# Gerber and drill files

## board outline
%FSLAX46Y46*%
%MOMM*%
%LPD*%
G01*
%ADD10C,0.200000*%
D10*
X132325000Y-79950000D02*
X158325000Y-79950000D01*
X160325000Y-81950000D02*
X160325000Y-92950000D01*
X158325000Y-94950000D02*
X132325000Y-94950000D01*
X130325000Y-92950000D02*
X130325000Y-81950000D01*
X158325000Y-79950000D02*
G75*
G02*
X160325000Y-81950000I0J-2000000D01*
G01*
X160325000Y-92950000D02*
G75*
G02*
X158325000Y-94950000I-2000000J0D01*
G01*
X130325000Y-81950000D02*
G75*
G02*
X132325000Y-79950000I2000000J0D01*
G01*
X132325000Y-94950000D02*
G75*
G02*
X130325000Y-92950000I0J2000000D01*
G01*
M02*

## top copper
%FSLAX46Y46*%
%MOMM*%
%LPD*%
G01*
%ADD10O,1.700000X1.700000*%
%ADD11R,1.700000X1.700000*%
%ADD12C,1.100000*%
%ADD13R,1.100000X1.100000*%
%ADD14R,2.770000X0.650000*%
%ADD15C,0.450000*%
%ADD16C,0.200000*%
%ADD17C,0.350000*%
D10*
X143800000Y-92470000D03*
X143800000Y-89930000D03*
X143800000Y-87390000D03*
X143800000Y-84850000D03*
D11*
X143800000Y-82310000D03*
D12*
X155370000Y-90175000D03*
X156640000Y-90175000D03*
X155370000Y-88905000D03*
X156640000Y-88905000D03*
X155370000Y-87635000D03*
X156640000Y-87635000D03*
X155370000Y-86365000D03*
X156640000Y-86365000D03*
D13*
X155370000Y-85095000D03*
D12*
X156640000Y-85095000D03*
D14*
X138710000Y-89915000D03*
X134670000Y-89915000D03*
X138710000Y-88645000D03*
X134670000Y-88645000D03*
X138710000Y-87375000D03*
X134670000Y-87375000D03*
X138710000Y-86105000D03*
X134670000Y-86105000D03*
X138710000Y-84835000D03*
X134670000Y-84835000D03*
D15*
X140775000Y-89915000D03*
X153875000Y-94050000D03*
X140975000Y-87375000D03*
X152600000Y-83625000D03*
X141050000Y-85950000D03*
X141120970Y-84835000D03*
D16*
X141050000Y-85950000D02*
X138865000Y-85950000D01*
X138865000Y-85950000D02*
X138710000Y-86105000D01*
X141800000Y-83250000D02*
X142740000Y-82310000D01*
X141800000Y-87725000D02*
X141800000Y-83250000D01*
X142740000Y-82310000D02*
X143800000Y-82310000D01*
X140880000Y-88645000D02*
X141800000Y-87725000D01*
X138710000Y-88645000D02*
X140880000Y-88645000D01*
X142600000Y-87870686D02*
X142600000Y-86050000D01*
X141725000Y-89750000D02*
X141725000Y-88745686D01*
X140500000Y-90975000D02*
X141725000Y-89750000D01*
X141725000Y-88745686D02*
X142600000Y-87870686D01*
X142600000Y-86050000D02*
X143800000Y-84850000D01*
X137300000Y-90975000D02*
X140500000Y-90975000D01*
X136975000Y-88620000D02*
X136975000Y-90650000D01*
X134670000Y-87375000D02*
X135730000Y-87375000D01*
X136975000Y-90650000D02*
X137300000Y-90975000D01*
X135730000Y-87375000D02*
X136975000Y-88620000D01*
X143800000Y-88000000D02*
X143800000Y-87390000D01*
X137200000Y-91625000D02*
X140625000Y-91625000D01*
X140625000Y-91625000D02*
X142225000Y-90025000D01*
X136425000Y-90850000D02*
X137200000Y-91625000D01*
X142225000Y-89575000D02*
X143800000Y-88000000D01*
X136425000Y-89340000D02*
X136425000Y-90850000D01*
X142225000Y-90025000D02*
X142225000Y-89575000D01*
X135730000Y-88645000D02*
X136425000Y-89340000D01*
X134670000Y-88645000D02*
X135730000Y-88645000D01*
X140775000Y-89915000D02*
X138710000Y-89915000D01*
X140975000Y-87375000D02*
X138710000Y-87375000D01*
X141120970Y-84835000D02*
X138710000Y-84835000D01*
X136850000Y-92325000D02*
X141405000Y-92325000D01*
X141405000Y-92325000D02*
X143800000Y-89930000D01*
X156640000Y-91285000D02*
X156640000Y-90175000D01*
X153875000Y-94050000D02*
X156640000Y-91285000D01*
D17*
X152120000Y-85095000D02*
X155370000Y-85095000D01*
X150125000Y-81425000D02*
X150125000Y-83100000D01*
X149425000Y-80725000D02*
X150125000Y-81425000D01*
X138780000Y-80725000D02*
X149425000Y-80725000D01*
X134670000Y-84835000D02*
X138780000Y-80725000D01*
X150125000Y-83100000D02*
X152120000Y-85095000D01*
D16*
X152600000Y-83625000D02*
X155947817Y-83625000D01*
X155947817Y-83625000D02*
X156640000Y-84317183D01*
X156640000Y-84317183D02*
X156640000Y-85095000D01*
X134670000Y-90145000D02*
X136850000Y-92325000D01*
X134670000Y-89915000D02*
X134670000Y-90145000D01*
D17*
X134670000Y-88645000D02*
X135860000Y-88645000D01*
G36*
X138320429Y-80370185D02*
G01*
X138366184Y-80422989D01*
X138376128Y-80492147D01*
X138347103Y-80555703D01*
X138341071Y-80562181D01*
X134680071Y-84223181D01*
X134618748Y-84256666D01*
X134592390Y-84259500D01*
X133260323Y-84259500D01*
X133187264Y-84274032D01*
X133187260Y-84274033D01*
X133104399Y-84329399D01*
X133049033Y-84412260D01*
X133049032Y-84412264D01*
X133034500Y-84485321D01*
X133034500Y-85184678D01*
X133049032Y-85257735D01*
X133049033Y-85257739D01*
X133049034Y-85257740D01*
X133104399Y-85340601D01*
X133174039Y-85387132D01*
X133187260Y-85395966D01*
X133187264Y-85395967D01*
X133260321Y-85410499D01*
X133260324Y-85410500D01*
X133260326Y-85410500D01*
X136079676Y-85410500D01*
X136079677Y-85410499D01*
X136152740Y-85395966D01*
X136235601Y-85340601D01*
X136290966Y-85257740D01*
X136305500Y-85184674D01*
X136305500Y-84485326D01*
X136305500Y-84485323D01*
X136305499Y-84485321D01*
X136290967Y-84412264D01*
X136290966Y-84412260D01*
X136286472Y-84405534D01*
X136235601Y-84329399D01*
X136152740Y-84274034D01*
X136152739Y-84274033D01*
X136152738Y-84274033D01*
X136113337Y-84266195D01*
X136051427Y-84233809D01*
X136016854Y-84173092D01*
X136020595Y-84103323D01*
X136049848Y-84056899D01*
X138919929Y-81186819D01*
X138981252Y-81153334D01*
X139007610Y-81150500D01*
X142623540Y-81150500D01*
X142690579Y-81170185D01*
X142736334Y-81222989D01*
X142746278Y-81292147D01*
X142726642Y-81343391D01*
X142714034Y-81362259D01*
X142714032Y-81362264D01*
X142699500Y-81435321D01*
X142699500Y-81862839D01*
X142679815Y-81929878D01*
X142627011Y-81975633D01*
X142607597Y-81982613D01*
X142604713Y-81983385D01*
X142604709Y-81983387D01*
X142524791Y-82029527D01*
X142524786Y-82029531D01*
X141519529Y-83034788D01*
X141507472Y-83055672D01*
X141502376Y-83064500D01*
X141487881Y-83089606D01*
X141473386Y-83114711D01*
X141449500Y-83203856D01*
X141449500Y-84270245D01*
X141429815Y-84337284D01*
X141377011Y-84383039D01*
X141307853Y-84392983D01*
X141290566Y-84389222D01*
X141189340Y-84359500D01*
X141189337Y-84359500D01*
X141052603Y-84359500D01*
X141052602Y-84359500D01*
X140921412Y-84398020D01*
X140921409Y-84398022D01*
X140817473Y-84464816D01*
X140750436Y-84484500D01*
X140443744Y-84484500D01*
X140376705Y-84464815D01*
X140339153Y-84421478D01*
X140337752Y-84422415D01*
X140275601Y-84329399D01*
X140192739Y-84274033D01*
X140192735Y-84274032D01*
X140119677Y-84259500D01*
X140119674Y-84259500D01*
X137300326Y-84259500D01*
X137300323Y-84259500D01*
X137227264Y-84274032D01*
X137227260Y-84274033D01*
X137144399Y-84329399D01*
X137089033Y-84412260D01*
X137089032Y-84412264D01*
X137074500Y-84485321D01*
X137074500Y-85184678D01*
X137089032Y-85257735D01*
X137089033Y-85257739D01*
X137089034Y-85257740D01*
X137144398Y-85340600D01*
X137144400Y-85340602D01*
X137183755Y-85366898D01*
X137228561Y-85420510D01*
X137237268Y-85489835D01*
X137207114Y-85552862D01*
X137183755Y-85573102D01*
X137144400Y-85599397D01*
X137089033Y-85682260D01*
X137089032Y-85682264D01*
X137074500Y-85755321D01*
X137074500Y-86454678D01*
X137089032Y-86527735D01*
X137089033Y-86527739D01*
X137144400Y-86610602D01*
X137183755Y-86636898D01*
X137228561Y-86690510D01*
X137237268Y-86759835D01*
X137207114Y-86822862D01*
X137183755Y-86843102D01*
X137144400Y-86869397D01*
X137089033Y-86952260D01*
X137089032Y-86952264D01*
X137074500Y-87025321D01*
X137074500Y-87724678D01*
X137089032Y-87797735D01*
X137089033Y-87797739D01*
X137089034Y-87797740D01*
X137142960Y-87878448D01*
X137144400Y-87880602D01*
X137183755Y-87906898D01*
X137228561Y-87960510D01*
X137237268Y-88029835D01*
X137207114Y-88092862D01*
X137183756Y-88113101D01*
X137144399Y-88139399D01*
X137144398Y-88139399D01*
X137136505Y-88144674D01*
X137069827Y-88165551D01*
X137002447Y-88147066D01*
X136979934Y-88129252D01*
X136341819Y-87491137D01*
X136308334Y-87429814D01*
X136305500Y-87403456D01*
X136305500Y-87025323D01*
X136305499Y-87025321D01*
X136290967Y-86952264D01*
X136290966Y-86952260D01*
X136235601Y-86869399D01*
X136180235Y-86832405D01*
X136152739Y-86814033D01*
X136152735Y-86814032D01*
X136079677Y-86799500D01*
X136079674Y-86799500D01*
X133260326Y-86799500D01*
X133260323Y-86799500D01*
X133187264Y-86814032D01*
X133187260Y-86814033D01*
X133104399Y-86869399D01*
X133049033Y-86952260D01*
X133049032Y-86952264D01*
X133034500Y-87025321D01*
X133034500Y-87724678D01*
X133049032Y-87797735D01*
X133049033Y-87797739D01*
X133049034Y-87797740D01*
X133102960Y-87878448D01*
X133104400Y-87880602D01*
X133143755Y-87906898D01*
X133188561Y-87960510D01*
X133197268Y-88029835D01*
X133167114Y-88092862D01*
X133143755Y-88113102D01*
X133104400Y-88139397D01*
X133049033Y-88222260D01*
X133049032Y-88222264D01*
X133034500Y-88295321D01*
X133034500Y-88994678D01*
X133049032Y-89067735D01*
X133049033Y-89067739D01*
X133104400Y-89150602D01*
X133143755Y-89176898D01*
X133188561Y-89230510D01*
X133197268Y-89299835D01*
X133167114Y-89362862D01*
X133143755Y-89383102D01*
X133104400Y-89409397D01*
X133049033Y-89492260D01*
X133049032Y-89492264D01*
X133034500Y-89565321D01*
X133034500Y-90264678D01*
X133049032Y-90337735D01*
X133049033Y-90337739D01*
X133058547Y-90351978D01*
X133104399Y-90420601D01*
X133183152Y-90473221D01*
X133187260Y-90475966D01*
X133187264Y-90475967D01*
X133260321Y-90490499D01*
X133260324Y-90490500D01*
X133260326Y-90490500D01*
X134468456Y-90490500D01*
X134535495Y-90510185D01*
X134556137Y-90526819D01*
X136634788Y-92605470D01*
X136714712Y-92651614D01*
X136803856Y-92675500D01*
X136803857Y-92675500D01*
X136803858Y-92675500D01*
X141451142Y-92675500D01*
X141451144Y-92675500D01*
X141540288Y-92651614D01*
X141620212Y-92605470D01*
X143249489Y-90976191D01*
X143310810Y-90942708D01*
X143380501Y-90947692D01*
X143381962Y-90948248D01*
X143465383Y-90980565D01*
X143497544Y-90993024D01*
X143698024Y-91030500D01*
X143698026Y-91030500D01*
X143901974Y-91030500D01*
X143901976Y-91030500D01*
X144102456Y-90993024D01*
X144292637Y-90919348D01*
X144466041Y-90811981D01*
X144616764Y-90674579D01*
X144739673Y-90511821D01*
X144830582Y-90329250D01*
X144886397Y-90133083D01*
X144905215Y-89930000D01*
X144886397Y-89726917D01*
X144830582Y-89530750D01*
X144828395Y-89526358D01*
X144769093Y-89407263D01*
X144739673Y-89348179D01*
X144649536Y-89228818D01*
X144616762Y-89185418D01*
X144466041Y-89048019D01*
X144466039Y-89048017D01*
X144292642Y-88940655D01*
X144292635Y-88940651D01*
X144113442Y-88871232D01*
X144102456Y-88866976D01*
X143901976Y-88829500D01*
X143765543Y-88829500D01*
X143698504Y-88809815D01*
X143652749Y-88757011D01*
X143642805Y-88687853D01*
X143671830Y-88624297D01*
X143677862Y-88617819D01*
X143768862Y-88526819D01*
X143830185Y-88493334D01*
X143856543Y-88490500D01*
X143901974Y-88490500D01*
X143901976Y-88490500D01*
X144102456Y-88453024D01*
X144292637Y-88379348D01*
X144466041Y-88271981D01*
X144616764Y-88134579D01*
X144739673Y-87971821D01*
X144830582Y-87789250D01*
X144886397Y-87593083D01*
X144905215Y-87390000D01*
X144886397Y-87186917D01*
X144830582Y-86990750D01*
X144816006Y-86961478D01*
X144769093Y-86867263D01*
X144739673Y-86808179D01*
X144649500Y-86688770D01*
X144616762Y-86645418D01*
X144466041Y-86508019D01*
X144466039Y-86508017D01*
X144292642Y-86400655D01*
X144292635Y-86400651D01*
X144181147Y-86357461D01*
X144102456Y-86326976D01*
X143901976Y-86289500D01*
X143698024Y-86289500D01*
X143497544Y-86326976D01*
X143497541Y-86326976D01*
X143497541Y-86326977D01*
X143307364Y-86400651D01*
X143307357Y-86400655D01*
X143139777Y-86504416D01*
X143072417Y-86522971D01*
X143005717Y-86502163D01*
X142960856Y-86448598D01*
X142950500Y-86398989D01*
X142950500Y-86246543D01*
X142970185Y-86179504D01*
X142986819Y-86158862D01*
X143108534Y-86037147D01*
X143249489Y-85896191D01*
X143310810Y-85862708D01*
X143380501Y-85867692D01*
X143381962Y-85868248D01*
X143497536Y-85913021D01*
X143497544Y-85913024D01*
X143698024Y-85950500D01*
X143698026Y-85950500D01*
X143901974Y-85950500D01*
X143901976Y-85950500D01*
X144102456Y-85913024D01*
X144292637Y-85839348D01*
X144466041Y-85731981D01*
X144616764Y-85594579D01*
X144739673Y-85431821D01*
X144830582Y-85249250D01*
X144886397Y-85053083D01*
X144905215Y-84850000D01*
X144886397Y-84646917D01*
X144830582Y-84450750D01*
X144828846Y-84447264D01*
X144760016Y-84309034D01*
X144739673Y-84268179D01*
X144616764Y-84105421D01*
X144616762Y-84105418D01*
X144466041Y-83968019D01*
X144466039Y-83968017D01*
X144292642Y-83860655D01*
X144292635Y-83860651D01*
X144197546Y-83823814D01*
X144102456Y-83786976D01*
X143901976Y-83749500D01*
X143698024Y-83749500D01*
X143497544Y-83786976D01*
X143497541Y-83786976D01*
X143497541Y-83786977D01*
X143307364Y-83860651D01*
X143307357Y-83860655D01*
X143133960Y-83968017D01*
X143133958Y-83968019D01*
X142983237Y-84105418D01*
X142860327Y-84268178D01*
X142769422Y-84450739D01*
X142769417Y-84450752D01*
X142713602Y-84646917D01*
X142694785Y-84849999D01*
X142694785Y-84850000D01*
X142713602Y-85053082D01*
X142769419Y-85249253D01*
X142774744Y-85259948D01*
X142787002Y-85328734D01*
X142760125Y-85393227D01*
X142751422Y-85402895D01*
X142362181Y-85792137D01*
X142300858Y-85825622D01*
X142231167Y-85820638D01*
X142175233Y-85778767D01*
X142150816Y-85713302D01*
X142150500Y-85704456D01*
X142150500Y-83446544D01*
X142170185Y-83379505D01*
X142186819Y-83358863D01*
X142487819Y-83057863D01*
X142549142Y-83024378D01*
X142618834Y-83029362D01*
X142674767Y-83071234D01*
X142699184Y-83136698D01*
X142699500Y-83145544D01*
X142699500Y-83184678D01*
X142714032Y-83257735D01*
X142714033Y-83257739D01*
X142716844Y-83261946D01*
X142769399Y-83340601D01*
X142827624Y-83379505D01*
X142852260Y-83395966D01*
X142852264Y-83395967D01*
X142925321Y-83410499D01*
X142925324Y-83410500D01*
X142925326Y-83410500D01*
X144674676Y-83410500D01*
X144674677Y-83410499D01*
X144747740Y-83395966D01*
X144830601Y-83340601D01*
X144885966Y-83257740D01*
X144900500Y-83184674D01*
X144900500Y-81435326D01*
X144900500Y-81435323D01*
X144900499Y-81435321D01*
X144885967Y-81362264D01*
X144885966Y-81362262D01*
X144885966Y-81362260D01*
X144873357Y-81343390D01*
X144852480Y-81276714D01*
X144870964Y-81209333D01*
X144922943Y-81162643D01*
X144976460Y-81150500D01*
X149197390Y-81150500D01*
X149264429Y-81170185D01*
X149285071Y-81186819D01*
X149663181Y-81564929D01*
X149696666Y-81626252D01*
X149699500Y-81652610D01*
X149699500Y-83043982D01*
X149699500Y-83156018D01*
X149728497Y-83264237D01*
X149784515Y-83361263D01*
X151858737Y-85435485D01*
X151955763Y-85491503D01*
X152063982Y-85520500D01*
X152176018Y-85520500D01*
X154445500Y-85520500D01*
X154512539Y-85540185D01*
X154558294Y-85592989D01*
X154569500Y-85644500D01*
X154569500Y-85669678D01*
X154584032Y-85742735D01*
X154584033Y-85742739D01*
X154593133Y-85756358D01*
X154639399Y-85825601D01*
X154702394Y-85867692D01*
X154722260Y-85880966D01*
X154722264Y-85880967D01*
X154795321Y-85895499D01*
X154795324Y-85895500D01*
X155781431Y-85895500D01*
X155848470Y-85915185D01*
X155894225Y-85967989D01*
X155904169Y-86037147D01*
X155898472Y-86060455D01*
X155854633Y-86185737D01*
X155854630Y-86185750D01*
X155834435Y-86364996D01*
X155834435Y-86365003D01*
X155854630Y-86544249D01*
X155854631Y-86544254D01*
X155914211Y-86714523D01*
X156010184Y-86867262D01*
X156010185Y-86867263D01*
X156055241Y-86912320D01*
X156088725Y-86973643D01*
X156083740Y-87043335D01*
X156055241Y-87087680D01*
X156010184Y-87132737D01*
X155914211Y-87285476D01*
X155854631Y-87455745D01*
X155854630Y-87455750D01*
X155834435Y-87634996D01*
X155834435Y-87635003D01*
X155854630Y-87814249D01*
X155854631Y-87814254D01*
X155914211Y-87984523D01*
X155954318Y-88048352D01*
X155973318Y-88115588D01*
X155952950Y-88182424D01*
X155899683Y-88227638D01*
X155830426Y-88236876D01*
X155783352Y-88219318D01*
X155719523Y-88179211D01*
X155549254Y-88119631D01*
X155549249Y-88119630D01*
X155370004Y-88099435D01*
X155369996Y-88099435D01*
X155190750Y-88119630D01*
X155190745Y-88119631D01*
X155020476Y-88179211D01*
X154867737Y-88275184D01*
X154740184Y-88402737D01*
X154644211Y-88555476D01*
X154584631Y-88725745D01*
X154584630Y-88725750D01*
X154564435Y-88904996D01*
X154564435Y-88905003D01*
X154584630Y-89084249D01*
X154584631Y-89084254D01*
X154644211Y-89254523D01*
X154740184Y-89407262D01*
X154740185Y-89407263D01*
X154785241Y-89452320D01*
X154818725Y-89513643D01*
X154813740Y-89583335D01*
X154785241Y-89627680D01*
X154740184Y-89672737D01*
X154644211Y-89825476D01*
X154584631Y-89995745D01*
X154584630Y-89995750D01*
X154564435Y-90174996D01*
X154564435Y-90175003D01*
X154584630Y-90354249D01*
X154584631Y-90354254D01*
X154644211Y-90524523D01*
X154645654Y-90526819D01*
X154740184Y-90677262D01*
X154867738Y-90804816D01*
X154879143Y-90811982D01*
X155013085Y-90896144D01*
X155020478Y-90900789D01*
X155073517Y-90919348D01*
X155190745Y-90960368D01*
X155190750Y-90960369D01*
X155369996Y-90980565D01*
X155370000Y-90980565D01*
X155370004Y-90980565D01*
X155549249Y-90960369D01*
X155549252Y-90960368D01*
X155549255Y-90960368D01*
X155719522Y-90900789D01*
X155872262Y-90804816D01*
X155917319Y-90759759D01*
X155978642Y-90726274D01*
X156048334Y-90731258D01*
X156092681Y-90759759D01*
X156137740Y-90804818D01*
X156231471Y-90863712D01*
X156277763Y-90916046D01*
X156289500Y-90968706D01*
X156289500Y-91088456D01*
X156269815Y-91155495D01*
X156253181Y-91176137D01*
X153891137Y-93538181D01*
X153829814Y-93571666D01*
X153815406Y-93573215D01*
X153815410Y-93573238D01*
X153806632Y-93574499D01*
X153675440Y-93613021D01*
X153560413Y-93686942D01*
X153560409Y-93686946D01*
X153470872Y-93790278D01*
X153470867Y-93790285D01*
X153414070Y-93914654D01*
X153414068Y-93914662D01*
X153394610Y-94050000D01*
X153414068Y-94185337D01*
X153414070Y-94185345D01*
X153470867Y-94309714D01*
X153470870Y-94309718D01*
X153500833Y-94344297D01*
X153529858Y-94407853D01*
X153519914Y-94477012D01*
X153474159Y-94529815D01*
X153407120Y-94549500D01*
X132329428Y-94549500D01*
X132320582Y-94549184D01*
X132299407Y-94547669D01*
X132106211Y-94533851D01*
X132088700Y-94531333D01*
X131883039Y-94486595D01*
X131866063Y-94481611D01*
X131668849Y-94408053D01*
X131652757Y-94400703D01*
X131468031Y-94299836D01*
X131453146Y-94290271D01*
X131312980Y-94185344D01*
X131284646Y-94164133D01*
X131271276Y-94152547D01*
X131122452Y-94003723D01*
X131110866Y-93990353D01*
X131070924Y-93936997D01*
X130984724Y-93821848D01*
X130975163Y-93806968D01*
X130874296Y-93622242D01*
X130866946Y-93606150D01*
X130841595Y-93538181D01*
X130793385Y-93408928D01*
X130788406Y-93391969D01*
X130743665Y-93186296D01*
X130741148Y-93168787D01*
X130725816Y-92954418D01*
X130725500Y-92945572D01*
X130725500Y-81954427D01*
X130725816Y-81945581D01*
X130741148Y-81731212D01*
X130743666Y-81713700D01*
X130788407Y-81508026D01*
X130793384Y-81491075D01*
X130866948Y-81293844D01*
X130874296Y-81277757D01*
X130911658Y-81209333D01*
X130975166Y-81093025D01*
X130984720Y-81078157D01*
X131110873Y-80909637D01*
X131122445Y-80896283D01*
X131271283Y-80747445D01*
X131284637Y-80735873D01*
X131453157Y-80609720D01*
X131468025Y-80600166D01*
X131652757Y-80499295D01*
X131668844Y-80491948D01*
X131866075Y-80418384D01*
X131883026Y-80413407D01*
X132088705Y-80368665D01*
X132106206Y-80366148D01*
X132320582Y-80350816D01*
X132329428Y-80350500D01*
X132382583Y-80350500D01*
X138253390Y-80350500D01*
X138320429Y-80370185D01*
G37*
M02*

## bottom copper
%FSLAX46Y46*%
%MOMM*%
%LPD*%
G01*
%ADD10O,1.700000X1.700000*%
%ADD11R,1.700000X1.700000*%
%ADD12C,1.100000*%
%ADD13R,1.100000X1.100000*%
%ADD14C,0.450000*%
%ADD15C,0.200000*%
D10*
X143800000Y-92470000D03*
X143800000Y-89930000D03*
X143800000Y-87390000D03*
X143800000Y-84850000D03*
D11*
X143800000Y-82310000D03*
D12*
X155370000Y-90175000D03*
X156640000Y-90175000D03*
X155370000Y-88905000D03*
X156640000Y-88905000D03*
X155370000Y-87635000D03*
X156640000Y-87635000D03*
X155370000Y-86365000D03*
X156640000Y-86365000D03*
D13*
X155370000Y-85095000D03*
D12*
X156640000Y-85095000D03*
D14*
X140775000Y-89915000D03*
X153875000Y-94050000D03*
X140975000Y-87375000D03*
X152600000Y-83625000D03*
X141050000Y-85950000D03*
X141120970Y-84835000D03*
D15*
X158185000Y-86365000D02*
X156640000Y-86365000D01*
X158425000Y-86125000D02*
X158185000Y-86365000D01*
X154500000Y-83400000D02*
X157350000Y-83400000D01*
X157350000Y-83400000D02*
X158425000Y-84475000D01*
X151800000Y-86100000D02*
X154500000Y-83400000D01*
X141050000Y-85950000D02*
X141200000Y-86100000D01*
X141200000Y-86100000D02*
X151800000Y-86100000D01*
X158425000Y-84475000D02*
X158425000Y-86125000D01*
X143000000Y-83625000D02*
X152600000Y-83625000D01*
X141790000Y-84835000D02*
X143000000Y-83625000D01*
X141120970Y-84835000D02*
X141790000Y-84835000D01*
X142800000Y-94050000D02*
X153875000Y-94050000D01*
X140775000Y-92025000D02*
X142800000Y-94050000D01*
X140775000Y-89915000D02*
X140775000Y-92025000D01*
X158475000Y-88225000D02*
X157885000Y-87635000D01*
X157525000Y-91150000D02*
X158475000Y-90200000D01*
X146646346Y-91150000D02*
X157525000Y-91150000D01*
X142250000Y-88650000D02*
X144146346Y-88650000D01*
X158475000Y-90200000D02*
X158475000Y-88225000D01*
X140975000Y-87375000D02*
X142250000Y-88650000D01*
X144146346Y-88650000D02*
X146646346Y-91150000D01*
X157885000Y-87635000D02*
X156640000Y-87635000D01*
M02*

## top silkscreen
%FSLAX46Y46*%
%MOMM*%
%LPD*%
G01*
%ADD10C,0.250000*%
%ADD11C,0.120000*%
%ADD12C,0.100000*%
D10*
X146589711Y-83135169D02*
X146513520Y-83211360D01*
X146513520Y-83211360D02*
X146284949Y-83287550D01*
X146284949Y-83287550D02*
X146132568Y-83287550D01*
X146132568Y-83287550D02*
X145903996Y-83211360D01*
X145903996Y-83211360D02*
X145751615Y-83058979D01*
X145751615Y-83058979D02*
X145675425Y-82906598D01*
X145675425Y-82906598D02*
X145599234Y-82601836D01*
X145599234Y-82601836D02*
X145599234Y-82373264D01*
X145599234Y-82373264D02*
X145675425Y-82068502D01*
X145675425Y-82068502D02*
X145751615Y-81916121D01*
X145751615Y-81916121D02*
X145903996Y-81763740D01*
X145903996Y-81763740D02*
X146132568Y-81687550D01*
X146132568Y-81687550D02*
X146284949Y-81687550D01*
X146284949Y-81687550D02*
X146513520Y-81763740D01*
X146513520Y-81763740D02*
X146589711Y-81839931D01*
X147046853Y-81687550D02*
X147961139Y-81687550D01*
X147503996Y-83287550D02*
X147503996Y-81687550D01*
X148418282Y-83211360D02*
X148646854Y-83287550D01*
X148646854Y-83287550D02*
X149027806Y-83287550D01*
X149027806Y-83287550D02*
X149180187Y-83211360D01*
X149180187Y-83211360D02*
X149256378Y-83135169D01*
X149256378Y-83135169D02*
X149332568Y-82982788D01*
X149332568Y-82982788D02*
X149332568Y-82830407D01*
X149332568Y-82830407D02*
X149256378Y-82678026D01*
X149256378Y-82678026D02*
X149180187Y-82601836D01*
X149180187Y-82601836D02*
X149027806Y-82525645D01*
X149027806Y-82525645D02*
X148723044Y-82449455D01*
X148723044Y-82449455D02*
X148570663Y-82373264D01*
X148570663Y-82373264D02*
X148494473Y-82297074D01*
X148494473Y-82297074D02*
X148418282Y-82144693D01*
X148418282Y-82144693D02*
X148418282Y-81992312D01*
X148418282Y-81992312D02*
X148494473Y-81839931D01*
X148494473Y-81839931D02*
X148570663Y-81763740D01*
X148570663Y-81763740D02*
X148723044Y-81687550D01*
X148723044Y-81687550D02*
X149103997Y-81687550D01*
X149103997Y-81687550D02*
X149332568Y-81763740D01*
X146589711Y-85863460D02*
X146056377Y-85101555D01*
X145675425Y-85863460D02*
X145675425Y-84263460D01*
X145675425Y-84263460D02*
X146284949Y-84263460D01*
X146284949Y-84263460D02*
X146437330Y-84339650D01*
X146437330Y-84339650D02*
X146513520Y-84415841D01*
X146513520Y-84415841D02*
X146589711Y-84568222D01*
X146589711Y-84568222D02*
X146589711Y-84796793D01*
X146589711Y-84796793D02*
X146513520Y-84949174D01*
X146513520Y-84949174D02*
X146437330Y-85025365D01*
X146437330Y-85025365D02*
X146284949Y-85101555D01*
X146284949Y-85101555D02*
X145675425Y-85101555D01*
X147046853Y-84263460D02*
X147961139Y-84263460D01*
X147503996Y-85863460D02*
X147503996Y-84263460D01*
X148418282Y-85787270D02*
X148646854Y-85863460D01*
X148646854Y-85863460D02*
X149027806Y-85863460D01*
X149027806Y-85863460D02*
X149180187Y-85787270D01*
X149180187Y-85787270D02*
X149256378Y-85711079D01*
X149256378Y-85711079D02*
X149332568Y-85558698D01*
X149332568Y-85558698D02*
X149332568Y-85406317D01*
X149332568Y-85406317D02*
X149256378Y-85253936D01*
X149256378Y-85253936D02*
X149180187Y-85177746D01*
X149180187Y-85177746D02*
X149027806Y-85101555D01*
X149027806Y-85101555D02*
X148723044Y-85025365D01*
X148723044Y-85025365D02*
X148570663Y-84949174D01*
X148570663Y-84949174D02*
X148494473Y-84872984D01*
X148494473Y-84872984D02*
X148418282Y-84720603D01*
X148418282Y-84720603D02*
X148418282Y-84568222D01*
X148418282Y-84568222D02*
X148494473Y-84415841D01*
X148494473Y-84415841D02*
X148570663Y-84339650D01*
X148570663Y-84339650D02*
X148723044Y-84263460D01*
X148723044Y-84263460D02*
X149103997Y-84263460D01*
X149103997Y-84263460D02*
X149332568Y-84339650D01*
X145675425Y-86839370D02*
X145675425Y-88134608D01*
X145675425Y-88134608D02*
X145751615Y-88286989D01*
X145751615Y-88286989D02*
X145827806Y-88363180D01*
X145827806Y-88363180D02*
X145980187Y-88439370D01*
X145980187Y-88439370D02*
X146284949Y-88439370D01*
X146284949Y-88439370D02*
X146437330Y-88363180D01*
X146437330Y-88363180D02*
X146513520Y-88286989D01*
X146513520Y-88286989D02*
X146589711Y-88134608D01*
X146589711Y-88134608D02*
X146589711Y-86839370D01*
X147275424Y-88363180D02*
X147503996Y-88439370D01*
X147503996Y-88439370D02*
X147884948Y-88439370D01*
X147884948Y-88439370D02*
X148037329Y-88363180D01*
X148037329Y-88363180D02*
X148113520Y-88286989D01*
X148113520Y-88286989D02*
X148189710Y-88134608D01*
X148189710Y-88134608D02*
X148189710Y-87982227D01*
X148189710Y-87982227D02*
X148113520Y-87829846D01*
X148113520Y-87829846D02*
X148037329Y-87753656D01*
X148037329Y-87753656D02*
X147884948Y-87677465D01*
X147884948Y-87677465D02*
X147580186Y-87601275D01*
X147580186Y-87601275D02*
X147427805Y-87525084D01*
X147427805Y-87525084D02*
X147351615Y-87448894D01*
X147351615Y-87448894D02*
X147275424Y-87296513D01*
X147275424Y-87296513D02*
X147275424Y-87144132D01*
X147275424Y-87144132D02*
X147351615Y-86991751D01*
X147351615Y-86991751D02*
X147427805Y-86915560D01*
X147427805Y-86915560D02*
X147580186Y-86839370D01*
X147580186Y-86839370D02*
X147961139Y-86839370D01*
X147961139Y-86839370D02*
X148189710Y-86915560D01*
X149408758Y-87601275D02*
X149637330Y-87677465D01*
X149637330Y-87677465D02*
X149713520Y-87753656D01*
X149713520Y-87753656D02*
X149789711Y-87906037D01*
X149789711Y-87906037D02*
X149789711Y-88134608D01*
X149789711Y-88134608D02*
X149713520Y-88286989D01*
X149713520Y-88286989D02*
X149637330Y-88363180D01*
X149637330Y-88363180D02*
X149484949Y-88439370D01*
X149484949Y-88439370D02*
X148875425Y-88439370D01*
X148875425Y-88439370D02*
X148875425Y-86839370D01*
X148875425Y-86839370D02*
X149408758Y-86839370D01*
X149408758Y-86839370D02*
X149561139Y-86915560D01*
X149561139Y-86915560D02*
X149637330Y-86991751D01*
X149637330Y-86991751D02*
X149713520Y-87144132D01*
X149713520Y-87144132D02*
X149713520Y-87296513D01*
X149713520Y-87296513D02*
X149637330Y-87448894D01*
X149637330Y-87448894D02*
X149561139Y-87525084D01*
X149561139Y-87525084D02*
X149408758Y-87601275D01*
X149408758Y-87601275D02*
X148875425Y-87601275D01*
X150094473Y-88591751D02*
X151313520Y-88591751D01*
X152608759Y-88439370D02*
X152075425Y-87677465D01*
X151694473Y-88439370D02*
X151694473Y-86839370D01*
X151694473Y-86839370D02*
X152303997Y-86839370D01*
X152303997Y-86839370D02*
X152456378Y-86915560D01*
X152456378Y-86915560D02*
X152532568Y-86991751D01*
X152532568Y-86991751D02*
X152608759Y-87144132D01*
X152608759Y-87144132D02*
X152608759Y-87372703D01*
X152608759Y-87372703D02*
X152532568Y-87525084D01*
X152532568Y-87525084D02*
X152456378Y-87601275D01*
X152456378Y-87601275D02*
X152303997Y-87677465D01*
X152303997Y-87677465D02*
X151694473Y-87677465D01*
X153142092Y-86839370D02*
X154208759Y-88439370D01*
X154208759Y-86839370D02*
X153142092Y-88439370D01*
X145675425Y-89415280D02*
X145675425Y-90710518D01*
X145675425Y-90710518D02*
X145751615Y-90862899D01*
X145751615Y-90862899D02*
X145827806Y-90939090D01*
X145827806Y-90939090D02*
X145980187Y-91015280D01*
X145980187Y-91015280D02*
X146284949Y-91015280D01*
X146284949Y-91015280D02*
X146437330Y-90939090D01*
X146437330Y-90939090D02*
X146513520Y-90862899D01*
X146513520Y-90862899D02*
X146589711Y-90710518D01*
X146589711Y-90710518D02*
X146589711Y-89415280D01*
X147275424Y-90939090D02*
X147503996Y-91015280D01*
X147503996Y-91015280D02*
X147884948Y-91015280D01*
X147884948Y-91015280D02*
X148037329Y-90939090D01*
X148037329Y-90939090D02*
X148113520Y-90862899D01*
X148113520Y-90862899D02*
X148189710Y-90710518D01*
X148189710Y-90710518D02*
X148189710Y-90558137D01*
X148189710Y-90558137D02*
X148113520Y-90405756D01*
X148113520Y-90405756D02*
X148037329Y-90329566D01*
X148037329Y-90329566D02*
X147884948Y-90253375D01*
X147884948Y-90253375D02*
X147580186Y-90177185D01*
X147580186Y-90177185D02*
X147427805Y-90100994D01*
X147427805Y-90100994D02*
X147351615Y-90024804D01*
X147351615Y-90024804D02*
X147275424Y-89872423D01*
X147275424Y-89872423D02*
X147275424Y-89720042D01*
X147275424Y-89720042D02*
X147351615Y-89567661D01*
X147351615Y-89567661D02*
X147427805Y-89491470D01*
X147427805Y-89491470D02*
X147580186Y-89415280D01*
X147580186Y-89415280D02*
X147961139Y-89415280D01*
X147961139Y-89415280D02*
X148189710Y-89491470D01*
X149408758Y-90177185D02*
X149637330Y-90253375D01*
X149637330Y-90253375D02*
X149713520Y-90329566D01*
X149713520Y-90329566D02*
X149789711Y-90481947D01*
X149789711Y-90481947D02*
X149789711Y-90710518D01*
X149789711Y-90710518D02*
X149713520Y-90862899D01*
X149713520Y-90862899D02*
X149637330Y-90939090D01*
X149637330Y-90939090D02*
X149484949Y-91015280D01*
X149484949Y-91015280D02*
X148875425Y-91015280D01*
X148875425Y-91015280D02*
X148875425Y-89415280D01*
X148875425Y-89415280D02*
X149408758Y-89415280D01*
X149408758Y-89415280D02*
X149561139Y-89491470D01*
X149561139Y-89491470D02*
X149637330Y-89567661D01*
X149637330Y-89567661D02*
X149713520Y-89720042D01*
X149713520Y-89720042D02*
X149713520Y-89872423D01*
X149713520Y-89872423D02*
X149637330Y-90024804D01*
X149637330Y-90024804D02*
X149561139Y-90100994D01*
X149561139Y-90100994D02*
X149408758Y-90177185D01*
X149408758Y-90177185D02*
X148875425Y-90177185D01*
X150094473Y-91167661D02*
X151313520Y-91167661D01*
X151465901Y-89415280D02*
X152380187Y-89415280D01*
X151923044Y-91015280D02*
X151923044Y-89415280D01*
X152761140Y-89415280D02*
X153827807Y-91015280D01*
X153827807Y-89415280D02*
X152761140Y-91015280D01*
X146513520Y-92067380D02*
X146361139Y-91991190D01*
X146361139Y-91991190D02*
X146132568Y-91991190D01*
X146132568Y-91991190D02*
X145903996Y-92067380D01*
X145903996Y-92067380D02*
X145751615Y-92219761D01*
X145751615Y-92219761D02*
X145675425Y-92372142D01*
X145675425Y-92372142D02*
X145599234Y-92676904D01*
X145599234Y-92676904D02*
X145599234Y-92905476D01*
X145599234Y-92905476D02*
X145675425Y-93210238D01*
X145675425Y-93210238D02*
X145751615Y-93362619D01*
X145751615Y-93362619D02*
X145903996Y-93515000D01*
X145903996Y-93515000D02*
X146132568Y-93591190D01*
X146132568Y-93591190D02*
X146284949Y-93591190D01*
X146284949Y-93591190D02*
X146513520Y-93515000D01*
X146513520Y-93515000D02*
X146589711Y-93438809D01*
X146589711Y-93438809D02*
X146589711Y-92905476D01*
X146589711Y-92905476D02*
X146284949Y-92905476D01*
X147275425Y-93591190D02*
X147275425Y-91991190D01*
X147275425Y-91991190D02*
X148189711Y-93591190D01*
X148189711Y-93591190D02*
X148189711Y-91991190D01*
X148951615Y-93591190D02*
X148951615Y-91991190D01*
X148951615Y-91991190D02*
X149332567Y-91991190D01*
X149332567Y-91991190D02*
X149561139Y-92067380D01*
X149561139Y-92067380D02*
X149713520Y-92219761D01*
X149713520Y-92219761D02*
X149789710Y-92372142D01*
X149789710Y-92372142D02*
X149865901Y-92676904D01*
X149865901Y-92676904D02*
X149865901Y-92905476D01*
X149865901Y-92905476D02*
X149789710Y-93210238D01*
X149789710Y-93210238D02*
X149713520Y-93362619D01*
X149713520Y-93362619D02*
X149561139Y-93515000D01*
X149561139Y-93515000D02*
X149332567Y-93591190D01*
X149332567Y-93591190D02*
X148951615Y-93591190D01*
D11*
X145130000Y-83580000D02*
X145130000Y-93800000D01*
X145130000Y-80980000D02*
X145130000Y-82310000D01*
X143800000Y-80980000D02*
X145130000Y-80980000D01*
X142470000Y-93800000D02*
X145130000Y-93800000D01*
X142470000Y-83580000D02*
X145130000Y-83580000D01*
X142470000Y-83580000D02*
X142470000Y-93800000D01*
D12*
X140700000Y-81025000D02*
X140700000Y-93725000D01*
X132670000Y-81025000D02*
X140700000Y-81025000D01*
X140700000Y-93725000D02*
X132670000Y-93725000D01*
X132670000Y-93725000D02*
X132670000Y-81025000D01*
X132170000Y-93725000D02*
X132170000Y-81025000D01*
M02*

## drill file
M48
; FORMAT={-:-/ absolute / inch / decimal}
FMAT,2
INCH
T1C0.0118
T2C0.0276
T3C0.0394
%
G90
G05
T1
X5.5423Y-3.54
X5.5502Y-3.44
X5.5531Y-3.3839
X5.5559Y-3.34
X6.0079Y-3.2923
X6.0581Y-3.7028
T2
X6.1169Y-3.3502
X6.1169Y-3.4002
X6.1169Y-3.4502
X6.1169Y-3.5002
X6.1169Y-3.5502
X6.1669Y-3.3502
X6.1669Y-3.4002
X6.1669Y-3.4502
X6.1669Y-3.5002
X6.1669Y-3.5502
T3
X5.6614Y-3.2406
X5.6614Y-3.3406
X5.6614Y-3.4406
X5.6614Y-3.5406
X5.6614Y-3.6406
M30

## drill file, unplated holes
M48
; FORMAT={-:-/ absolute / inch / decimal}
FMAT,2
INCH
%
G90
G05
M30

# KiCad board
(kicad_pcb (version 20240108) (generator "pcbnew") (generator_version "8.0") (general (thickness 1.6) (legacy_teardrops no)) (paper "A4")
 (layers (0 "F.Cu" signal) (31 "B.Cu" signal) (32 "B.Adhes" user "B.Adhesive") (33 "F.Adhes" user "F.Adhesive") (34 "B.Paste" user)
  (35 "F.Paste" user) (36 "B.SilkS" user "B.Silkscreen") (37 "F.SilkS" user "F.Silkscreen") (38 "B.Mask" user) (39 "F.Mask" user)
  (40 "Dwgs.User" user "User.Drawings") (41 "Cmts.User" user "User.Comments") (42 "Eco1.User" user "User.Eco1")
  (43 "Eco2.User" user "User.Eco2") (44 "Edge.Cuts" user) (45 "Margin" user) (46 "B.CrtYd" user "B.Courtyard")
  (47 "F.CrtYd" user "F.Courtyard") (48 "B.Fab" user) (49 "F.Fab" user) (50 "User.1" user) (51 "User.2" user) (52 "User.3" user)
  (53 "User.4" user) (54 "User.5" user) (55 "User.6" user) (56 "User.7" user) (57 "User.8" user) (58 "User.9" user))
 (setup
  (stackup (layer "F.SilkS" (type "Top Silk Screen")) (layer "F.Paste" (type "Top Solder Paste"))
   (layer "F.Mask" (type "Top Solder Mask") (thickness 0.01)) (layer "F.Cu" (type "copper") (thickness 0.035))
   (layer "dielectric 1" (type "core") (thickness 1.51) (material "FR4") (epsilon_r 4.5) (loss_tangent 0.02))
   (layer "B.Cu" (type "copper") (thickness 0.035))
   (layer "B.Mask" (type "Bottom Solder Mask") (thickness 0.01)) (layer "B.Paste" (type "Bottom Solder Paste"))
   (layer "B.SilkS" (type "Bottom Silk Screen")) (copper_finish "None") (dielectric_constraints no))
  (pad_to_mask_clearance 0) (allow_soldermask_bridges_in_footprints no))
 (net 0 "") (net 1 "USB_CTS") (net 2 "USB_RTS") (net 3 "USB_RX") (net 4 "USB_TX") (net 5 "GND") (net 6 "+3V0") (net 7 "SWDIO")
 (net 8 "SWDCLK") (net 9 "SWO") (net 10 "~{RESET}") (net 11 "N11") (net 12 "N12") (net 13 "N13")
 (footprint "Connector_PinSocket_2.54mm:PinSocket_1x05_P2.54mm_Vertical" (layer "F.Cu") (at 143.8 82.31)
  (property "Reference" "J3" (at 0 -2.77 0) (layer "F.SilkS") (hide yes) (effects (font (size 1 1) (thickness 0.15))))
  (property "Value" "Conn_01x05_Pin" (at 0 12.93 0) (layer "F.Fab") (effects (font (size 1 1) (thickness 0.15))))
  (fp_line (start -1.33 1.27) (end -1.33 11.49) (stroke (width 0.12) (type solid)) (layer "F.SilkS"))
  (fp_line (start -1.33 1.27) (end 1.33 1.27) (stroke (width 0.12) (type solid)) (layer "F.SilkS"))
  (fp_line (start -1.33 11.49) (end 1.33 11.49) (stroke (width 0.12) (type solid)) (layer "F.SilkS"))
  (fp_line (start 0 -1.33) (end 1.33 -1.33) (stroke (width 0.12) (type solid)) (layer "F.SilkS"))
  (fp_line (start 1.33 -1.33) (end 1.33 0) (stroke (width 0.12) (type solid)) (layer "F.SilkS"))
  (fp_line (start 1.33 1.27) (end 1.33 11.49) (stroke (width 0.12) (type solid)) (layer "F.SilkS"))
  (pad "1" thru_hole rect (at 0 0) (size 1.7 1.7) (drill 1) (layers "*.Cu" "*.Mask") (remove_unused_layers no) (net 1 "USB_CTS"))
  (pad "2" thru_hole oval (at 0 2.54) (size 1.7 1.7) (drill 1) (layers "*.Cu" "*.Mask") (remove_unused_layers no) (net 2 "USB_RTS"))
  (pad "3" thru_hole oval (at 0 5.08) (size 1.7 1.7) (drill 1) (layers "*.Cu" "*.Mask") (remove_unused_layers no) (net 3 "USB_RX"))
  (pad "4" thru_hole oval (at 0 7.62) (size 1.7 1.7) (drill 1) (layers "*.Cu" "*.Mask") (remove_unused_layers no) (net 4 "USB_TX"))
  (pad "5" thru_hole oval (at 0 10.16) (size 1.7 1.7) (drill 1) (layers "*.Cu" "*.Mask") (remove_unused_layers no) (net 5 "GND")))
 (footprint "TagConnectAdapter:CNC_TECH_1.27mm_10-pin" (layer "F.Cu") (at 136.67 87.415 90)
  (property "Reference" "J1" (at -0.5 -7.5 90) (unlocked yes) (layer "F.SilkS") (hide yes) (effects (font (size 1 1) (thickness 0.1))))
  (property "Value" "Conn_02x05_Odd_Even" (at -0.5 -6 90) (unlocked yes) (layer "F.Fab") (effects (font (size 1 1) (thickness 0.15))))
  (fp_line (start -6.31 -4.5) (end 6.39 -4.5) (stroke (width 0.1) (type default)) (layer "F.SilkS"))
  (fp_line (start 6.39 -4) (end 6.39 4.03) (stroke (width 0.1) (type default)) (layer "F.SilkS"))
  (fp_line (start -6.31 -4) (end 6.39 -4) (stroke (width 0.1) (type default)) (layer "F.SilkS"))
  (fp_line (start 6.39 4.03) (end -6.31 4.03) (stroke (width 0.1) (type default)) (layer "F.SilkS"))
  (fp_line (start -6.31 4.03) (end -6.31 -4) (stroke (width 0.1) (type default)) (layer "F.SilkS"))
  (pad "1" smd rect (at 2.58 -2 90) (size 0.65 2.77) (layers "F.Cu" "F.Paste" "F.Mask") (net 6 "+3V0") (thermal_bridge_angle 45))
  (pad "2" smd rect (at 2.58 2.04 90) (size 0.65 2.77) (layers "F.Cu" "F.Paste" "F.Mask") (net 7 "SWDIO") (thermal_bridge_angle 45))
  (pad "3" smd rect (at 1.31 -2 90) (size 0.65 2.77) (layers "F.Cu" "F.Paste" "F.Mask") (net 5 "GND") (thermal_bridge_angle 45))
  (pad "4" smd rect (at 1.31 2.04 90) (size 0.65 2.77) (layers "F.Cu" "F.Paste" "F.Mask") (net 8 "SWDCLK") (thermal_bridge_angle 45))
  (pad "5" smd rect (at 0.04 -2 90) (size 0.65 2.77) (layers "F.Cu" "F.Paste" "F.Mask") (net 2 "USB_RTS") (thermal_bridge_angle 45))
  (pad "6" smd rect (at 0.04 2.04 90) (size 0.65 2.77) (layers "F.Cu" "F.Paste" "F.Mask") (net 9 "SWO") (thermal_bridge_angle 45))
  (pad "7" smd rect (at -1.23 -2 90) (size 0.65 2.77) (layers "F.Cu" "F.Paste" "F.Mask") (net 3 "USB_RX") (thermal_bridge_angle 45))
  (pad "8" smd rect (at -1.23 2.04 90) (size 0.65 2.77) (layers "F.Cu" "F.Paste" "F.Mask") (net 1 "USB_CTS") (thermal_bridge_angle 45))
  (pad "9" smd rect (at -2.5 -2 90) (size 0.65 2.77) (layers "F.Cu" "F.Paste" "F.Mask") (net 4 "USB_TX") (thermal_bridge_angle 45))
  (pad "10" smd rect (at -2.5 2.04 90) (size 0.65 2.77) (layers "F.Cu" "F.Paste" "F.Mask") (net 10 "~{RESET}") (thermal_bridge_angle 45)))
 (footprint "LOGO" (layer "B.Cu") (at 138.95 87.3 90)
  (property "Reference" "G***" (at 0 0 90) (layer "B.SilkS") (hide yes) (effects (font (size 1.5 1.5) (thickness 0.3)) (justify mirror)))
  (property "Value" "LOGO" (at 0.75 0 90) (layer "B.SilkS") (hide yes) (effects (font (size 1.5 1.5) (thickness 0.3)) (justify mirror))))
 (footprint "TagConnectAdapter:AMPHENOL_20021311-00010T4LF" (layer "B.Cu") (at 156.005 87.635 90)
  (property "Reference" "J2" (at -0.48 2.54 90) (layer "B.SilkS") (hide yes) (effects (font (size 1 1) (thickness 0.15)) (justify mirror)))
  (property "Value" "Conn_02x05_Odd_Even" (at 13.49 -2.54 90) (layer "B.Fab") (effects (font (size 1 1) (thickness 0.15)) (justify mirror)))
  (pad "1" thru_hole rect (at 2.54 -0.635 90) (size 1.1 1.1) (drill 0.7) (layers "*.Cu" "*.Mask") (remove_unused_layers no) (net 6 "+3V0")
   (solder_mask_margin 0.102))
  (pad "2" thru_hole circle (at 2.54 0.635 90) (size 1.1 1.1) (drill 0.7) (layers "*.Cu" "*.Mask") (remove_unused_layers no) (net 7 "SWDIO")
   (solder_mask_margin 0.102))
  (pad "3" thru_hole circle (at 1.27 -0.635 90) (size 1.1 1.1) (drill 0.7) (layers "*.Cu" "*.Mask") (remove_unused_layers no) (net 5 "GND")
   (solder_mask_margin 0.102))
  (pad "4" thru_hole circle (at 1.27 0.635 90) (size 1.1 1.1) (drill 0.7) (layers "*.Cu" "*.Mask") (remove_unused_layers no)
   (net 8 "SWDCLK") (solder_mask_margin 0.102))
  (pad "5" thru_hole circle (at 0 -0.635 90) (size 1.1 1.1) (drill 0.7) (layers "*.Cu" "*.Mask") (remove_unused_layers no) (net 5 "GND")
   (solder_mask_margin 0.102))
  (pad "6" thru_hole circle (at 0 0.635 90) (size 1.1 1.1) (drill 0.7) (layers "*.Cu" "*.Mask") (remove_unused_layers no) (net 9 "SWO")
   (solder_mask_margin 0.102))
  (pad "7" thru_hole circle (at -1.27 -0.635 90) (size 1.1 1.1) (drill 0.7) (layers "*.Cu" "*.Mask") (remove_unused_layers no)
   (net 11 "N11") (solder_mask_margin 0.102))
  (pad "8" thru_hole circle (at -1.27 0.635 90) (size 1.1 1.1) (drill 0.7) (layers "*.Cu" "*.Mask") (remove_unused_layers no) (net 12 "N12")
   (solder_mask_margin 0.102))
  (pad "9" thru_hole circle (at -2.54 -0.635 90) (size 1.1 1.1) (drill 0.7) (layers "*.Cu" "*.Mask") (remove_unused_layers no)
   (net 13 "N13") (solder_mask_margin 0.102))
  (pad "10" thru_hole circle (at -2.54 0.635 90) (size 1.1 1.1) (drill 0.7) (layers "*.Cu" "*.Mask") (remove_unused_layers no)
   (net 10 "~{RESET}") (solder_mask_margin 0.102)))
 (gr_arc (start 132.325 94.95) (mid 130.910786 94.364214) (end 130.325 92.95) (stroke (width 0.2) (type default)) (layer "Edge.Cuts"))
 (gr_arc (start 160.325 92.95) (mid 159.739214 94.364214) (end 158.325 94.95) (stroke (width 0.2) (type default)) (layer "Edge.Cuts"))
 (gr_line (start 130.325 92.95) (end 130.325 81.95) (stroke (width 0.2) (type default)) (layer "Edge.Cuts"))
 (gr_line (start 132.325 79.95) (end 158.325 79.95) (stroke (width 0.2) (type default)) (layer "Edge.Cuts"))
 (gr_arc (start 130.325 81.95) (mid 130.910786 80.535786) (end 132.325 79.95) (stroke (width 0.2) (type default)) (layer "Edge.Cuts"))
 (gr_line (start 158.325 94.95) (end 132.325 94.95) (stroke (width 0.2) (type default)) (layer "Edge.Cuts"))
 (gr_arc (start 158.325 79.95) (mid 159.739214 80.535786) (end 160.325 81.95) (stroke (width 0.2) (type default)) (layer "Edge.Cuts"))
 (gr_line (start 160.325 81.95) (end 160.325 92.95) (stroke (width 0.2) (type default)) (layer "Edge.Cuts"))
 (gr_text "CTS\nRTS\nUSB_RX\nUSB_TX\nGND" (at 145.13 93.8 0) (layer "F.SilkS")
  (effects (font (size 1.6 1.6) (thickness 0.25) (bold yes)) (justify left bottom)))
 (segment (start 138.78 80.725) (end 149.425 80.725) (width 0.35) (layer "F.Cu") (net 6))
 (segment (start 134.67 84.835) (end 138.78 80.725) (width 0.35) (layer "F.Cu") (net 6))
 (segment (start 152.12 85.095) (end 155.37 85.095) (width 0.35) (layer "F.Cu") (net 6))
 (segment (start 150.125 81.425) (end 150.125 83.1) (width 0.35) (layer "F.Cu") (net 6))
 (segment (start 149.425 80.725) (end 150.125 81.425) (width 0.35) (layer "F.Cu") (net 6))
 (segment (start 150.125 83.1) (end 152.12 85.095) (width 0.35) (layer "F.Cu") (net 6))
 (segment (start 134.67 89.915) (end 134.67 90.145) (width 0.2) (layer "F.Cu") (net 4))
 (segment (start 136.85 92.325) (end 141.405 92.325) (width 0.2) (layer "F.Cu") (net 4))
 (segment (start 134.67 90.145) (end 136.85 92.325) (width 0.2) (layer "F.Cu") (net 4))
 (segment (start 141.405 92.325) (end 143.8 89.93) (width 0.2) (layer "F.Cu") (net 4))
 (segment (start 153.875 94.05) (end 156.64 91.285) (width 0.2) (layer "F.Cu") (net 10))
 (segment (start 140.775 89.915) (end 138.71 89.915) (width 0.2) (layer "F.Cu") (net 10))
 (segment (start 156.64 91.285) (end 156.64 90.175) (width 0.2) (layer "F.Cu") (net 10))
 (via (at 140.775 89.915) (size 0.45) (drill 0.3) (layers "F.Cu" "B.Cu") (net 10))
 (via (at 153.875 94.05) (size 0.45) (drill 0.3) (layers "F.Cu" "B.Cu") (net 10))
 (segment (start 142.8 94.05) (end 153.875 94.05) (width 0.2) (layer "B.Cu") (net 10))
 (segment (start 140.775 89.915) (end 140.775 92.025) (width 0.2) (layer "B.Cu") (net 10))
 (segment (start 140.775 92.025) (end 142.8 94.05) (width 0.2) (layer "B.Cu") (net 10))
 (segment (start 156.64 84.317183) (end 156.64 85.095) (width 0.2) (layer "F.Cu") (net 7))
 (segment (start 141.12097 84.835) (end 138.71 84.835) (width 0.2) (layer "F.Cu") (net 7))
 (segment (start 155.947817 83.625) (end 156.64 84.317183) (width 0.2) (layer "F.Cu") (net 7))
 (segment (start 152.6 83.625) (end 155.947817 83.625) (width 0.2) (layer "F.Cu") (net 7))
 (via (at 152.6 83.625) (size 0.45) (drill 0.3) (layers "F.Cu" "B.Cu") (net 7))
 (via (at 141.12097 84.835) (size 0.45) (drill 0.3) (layers "F.Cu" "B.Cu") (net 7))
 (segment (start 143 83.625) (end 152.6 83.625) (width 0.2) (layer "B.Cu") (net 7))
 (segment (start 141.79 84.835) (end 143 83.625) (width 0.2) (layer "B.Cu") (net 7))
 (segment (start 141.12097 84.835) (end 141.79 84.835) (width 0.2) (layer "B.Cu") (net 7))
 (segment (start 134.67 87.375) (end 135.73 87.375) (width 0.2) (layer "F.Cu") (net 2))
 (segment (start 142.6 87.870686) (end 142.6 86.05) (width 0.2) (layer "F.Cu") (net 2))
 (segment (start 140.5 90.975) (end 141.725 89.75) (width 0.2) (layer "F.Cu") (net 2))
 (segment (start 141.725 88.745686) (end 142.6 87.870686) (width 0.2) (layer "F.Cu") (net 2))
 (segment (start 141.725 89.75) (end 141.725 88.745686) (width 0.2) (layer "F.Cu") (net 2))
 (segment (start 136.975 88.62) (end 136.975 90.65) (width 0.2) (layer "F.Cu") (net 2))
 (segment (start 142.6 86.05) (end 143.8 84.85) (width 0.2) (layer "F.Cu") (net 2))
 (segment (start 135.73 87.375) (end 136.975 88.62) (width 0.2) (layer "F.Cu") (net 2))
 (segment (start 136.975 90.65) (end 137.3 90.975) (width 0.2) (layer "F.Cu") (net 2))
 (segment (start 137.3 90.975) (end 140.5 90.975) (width 0.2) (layer "F.Cu") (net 2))
 (segment (start 140.975 87.375) (end 138.71 87.375) (width 0.2) (layer "F.Cu") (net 9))
 (via (at 140.975 87.375) (size 0.45) (drill 0.3) (layers "F.Cu" "B.Cu") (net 9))
 (segment (start 144.146346 88.65) (end 146.646346 91.15) (width 0.2) (layer "B.Cu") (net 9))
 (segment (start 142.25 88.65) (end 144.146346 88.65) (width 0.2) (layer "B.Cu") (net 9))
 (segment (start 158.475 90.2) (end 158.475 88.225) (width 0.2) (layer "B.Cu") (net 9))
 (segment (start 157.885 87.635) (end 156.64 87.635) (width 0.2) (layer "B.Cu") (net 9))
 (segment (start 158.475 88.225) (end 157.885 87.635) (width 0.2) (layer "B.Cu") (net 9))
 (segment (start 146.646346 91.15) (end 157.525 91.15) (width 0.2) (layer "B.Cu") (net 9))
 (segment (start 157.525 91.15) (end 158.475 90.2) (width 0.2) (layer "B.Cu") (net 9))
 (segment (start 140.975 87.375) (end 142.25 88.65) (width 0.2) (layer "B.Cu") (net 9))
 (segment (start 142.225 89.575) (end 143.8 88) (width 0.2) (layer "F.Cu") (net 3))
 (segment (start 134.67 88.645) (end 135.73 88.645) (width 0.2) (layer "F.Cu") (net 3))
 (segment (start 134.67 88.645) (end 135.86 88.645) (width 0.35) (layer "F.Cu") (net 3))
 (segment (start 143.8 88) (end 143.8 87.39) (width 0.2) (layer "F.Cu") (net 3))
 (segment (start 135.73 88.645) (end 136.425 89.34) (width 0.2) (layer "F.Cu") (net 3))
 (segment (start 136.425 90.85) (end 137.2 91.625) (width 0.2) (layer "F.Cu") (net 3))
 (segment (start 136.425 89.34) (end 136.425 90.85) (width 0.2) (layer "F.Cu") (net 3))
 (segment (start 142.225 90.025) (end 142.225 89.575) (width 0.2) (layer "F.Cu") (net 3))
 (segment (start 140.625 91.625) (end 142.225 90.025) (width 0.2) (layer "F.Cu") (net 3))
 (segment (start 137.2 91.625) (end 140.625 91.625) (width 0.2) (layer "F.Cu") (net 3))
 (segment (start 138.865 85.95) (end 138.71 86.105) (width 0.2) (layer "F.Cu") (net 8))
 (segment (start 141.05 85.95) (end 138.865 85.95) (width 0.2) (layer "F.Cu") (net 8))
 (via (at 141.05 85.95) (size 0.45) (drill 0.3) (layers "F.Cu" "B.Cu") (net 8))
 (segment (start 141.05 85.95) (end 141.2 86.1) (width 0.2) (layer "B.Cu") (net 8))
 (segment (start 158.425 86.125) (end 158.185 86.365) (width 0.2) (layer "B.Cu") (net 8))
 (segment (start 157.35 83.4) (end 158.425 84.475) (width 0.2) (layer "B.Cu") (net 8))
 (segment (start 151.8 86.1) (end 154.5 83.4) (width 0.2) (layer "B.Cu") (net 8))
 (segment (start 158.185 86.365) (end 156.64 86.365) (width 0.2) (layer "B.Cu") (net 8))
 (segment (start 141.2 86.1) (end 151.8 86.1) (width 0.2) (layer "B.Cu") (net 8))
 (segment (start 154.5 83.4) (end 157.35 83.4) (width 0.2) (layer "B.Cu") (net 8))
 (segment (start 158.425 84.475) (end 158.425 86.125) (width 0.2) (layer "B.Cu") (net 8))
 (segment (start 141.8 87.725) (end 141.8 83.25) (width 0.2) (layer "F.Cu") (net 1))
 (segment (start 142.74 82.31) (end 143.8 82.31) (width 0.2) (layer "F.Cu") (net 1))
 (segment (start 138.71 88.645) (end 140.88 88.645) (width 0.2) (layer "F.Cu") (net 1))
 (segment (start 140.88 88.645) (end 141.8 87.725) (width 0.2) (layer "F.Cu") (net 1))
 (segment (start 141.8 83.25) (end 142.74 82.31) (width 0.2) (layer "F.Cu") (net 1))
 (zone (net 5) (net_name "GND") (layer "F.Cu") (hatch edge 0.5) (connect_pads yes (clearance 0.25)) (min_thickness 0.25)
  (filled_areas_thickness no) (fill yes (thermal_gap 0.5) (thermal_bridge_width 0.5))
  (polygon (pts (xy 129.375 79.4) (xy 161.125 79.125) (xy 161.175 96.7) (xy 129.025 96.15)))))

